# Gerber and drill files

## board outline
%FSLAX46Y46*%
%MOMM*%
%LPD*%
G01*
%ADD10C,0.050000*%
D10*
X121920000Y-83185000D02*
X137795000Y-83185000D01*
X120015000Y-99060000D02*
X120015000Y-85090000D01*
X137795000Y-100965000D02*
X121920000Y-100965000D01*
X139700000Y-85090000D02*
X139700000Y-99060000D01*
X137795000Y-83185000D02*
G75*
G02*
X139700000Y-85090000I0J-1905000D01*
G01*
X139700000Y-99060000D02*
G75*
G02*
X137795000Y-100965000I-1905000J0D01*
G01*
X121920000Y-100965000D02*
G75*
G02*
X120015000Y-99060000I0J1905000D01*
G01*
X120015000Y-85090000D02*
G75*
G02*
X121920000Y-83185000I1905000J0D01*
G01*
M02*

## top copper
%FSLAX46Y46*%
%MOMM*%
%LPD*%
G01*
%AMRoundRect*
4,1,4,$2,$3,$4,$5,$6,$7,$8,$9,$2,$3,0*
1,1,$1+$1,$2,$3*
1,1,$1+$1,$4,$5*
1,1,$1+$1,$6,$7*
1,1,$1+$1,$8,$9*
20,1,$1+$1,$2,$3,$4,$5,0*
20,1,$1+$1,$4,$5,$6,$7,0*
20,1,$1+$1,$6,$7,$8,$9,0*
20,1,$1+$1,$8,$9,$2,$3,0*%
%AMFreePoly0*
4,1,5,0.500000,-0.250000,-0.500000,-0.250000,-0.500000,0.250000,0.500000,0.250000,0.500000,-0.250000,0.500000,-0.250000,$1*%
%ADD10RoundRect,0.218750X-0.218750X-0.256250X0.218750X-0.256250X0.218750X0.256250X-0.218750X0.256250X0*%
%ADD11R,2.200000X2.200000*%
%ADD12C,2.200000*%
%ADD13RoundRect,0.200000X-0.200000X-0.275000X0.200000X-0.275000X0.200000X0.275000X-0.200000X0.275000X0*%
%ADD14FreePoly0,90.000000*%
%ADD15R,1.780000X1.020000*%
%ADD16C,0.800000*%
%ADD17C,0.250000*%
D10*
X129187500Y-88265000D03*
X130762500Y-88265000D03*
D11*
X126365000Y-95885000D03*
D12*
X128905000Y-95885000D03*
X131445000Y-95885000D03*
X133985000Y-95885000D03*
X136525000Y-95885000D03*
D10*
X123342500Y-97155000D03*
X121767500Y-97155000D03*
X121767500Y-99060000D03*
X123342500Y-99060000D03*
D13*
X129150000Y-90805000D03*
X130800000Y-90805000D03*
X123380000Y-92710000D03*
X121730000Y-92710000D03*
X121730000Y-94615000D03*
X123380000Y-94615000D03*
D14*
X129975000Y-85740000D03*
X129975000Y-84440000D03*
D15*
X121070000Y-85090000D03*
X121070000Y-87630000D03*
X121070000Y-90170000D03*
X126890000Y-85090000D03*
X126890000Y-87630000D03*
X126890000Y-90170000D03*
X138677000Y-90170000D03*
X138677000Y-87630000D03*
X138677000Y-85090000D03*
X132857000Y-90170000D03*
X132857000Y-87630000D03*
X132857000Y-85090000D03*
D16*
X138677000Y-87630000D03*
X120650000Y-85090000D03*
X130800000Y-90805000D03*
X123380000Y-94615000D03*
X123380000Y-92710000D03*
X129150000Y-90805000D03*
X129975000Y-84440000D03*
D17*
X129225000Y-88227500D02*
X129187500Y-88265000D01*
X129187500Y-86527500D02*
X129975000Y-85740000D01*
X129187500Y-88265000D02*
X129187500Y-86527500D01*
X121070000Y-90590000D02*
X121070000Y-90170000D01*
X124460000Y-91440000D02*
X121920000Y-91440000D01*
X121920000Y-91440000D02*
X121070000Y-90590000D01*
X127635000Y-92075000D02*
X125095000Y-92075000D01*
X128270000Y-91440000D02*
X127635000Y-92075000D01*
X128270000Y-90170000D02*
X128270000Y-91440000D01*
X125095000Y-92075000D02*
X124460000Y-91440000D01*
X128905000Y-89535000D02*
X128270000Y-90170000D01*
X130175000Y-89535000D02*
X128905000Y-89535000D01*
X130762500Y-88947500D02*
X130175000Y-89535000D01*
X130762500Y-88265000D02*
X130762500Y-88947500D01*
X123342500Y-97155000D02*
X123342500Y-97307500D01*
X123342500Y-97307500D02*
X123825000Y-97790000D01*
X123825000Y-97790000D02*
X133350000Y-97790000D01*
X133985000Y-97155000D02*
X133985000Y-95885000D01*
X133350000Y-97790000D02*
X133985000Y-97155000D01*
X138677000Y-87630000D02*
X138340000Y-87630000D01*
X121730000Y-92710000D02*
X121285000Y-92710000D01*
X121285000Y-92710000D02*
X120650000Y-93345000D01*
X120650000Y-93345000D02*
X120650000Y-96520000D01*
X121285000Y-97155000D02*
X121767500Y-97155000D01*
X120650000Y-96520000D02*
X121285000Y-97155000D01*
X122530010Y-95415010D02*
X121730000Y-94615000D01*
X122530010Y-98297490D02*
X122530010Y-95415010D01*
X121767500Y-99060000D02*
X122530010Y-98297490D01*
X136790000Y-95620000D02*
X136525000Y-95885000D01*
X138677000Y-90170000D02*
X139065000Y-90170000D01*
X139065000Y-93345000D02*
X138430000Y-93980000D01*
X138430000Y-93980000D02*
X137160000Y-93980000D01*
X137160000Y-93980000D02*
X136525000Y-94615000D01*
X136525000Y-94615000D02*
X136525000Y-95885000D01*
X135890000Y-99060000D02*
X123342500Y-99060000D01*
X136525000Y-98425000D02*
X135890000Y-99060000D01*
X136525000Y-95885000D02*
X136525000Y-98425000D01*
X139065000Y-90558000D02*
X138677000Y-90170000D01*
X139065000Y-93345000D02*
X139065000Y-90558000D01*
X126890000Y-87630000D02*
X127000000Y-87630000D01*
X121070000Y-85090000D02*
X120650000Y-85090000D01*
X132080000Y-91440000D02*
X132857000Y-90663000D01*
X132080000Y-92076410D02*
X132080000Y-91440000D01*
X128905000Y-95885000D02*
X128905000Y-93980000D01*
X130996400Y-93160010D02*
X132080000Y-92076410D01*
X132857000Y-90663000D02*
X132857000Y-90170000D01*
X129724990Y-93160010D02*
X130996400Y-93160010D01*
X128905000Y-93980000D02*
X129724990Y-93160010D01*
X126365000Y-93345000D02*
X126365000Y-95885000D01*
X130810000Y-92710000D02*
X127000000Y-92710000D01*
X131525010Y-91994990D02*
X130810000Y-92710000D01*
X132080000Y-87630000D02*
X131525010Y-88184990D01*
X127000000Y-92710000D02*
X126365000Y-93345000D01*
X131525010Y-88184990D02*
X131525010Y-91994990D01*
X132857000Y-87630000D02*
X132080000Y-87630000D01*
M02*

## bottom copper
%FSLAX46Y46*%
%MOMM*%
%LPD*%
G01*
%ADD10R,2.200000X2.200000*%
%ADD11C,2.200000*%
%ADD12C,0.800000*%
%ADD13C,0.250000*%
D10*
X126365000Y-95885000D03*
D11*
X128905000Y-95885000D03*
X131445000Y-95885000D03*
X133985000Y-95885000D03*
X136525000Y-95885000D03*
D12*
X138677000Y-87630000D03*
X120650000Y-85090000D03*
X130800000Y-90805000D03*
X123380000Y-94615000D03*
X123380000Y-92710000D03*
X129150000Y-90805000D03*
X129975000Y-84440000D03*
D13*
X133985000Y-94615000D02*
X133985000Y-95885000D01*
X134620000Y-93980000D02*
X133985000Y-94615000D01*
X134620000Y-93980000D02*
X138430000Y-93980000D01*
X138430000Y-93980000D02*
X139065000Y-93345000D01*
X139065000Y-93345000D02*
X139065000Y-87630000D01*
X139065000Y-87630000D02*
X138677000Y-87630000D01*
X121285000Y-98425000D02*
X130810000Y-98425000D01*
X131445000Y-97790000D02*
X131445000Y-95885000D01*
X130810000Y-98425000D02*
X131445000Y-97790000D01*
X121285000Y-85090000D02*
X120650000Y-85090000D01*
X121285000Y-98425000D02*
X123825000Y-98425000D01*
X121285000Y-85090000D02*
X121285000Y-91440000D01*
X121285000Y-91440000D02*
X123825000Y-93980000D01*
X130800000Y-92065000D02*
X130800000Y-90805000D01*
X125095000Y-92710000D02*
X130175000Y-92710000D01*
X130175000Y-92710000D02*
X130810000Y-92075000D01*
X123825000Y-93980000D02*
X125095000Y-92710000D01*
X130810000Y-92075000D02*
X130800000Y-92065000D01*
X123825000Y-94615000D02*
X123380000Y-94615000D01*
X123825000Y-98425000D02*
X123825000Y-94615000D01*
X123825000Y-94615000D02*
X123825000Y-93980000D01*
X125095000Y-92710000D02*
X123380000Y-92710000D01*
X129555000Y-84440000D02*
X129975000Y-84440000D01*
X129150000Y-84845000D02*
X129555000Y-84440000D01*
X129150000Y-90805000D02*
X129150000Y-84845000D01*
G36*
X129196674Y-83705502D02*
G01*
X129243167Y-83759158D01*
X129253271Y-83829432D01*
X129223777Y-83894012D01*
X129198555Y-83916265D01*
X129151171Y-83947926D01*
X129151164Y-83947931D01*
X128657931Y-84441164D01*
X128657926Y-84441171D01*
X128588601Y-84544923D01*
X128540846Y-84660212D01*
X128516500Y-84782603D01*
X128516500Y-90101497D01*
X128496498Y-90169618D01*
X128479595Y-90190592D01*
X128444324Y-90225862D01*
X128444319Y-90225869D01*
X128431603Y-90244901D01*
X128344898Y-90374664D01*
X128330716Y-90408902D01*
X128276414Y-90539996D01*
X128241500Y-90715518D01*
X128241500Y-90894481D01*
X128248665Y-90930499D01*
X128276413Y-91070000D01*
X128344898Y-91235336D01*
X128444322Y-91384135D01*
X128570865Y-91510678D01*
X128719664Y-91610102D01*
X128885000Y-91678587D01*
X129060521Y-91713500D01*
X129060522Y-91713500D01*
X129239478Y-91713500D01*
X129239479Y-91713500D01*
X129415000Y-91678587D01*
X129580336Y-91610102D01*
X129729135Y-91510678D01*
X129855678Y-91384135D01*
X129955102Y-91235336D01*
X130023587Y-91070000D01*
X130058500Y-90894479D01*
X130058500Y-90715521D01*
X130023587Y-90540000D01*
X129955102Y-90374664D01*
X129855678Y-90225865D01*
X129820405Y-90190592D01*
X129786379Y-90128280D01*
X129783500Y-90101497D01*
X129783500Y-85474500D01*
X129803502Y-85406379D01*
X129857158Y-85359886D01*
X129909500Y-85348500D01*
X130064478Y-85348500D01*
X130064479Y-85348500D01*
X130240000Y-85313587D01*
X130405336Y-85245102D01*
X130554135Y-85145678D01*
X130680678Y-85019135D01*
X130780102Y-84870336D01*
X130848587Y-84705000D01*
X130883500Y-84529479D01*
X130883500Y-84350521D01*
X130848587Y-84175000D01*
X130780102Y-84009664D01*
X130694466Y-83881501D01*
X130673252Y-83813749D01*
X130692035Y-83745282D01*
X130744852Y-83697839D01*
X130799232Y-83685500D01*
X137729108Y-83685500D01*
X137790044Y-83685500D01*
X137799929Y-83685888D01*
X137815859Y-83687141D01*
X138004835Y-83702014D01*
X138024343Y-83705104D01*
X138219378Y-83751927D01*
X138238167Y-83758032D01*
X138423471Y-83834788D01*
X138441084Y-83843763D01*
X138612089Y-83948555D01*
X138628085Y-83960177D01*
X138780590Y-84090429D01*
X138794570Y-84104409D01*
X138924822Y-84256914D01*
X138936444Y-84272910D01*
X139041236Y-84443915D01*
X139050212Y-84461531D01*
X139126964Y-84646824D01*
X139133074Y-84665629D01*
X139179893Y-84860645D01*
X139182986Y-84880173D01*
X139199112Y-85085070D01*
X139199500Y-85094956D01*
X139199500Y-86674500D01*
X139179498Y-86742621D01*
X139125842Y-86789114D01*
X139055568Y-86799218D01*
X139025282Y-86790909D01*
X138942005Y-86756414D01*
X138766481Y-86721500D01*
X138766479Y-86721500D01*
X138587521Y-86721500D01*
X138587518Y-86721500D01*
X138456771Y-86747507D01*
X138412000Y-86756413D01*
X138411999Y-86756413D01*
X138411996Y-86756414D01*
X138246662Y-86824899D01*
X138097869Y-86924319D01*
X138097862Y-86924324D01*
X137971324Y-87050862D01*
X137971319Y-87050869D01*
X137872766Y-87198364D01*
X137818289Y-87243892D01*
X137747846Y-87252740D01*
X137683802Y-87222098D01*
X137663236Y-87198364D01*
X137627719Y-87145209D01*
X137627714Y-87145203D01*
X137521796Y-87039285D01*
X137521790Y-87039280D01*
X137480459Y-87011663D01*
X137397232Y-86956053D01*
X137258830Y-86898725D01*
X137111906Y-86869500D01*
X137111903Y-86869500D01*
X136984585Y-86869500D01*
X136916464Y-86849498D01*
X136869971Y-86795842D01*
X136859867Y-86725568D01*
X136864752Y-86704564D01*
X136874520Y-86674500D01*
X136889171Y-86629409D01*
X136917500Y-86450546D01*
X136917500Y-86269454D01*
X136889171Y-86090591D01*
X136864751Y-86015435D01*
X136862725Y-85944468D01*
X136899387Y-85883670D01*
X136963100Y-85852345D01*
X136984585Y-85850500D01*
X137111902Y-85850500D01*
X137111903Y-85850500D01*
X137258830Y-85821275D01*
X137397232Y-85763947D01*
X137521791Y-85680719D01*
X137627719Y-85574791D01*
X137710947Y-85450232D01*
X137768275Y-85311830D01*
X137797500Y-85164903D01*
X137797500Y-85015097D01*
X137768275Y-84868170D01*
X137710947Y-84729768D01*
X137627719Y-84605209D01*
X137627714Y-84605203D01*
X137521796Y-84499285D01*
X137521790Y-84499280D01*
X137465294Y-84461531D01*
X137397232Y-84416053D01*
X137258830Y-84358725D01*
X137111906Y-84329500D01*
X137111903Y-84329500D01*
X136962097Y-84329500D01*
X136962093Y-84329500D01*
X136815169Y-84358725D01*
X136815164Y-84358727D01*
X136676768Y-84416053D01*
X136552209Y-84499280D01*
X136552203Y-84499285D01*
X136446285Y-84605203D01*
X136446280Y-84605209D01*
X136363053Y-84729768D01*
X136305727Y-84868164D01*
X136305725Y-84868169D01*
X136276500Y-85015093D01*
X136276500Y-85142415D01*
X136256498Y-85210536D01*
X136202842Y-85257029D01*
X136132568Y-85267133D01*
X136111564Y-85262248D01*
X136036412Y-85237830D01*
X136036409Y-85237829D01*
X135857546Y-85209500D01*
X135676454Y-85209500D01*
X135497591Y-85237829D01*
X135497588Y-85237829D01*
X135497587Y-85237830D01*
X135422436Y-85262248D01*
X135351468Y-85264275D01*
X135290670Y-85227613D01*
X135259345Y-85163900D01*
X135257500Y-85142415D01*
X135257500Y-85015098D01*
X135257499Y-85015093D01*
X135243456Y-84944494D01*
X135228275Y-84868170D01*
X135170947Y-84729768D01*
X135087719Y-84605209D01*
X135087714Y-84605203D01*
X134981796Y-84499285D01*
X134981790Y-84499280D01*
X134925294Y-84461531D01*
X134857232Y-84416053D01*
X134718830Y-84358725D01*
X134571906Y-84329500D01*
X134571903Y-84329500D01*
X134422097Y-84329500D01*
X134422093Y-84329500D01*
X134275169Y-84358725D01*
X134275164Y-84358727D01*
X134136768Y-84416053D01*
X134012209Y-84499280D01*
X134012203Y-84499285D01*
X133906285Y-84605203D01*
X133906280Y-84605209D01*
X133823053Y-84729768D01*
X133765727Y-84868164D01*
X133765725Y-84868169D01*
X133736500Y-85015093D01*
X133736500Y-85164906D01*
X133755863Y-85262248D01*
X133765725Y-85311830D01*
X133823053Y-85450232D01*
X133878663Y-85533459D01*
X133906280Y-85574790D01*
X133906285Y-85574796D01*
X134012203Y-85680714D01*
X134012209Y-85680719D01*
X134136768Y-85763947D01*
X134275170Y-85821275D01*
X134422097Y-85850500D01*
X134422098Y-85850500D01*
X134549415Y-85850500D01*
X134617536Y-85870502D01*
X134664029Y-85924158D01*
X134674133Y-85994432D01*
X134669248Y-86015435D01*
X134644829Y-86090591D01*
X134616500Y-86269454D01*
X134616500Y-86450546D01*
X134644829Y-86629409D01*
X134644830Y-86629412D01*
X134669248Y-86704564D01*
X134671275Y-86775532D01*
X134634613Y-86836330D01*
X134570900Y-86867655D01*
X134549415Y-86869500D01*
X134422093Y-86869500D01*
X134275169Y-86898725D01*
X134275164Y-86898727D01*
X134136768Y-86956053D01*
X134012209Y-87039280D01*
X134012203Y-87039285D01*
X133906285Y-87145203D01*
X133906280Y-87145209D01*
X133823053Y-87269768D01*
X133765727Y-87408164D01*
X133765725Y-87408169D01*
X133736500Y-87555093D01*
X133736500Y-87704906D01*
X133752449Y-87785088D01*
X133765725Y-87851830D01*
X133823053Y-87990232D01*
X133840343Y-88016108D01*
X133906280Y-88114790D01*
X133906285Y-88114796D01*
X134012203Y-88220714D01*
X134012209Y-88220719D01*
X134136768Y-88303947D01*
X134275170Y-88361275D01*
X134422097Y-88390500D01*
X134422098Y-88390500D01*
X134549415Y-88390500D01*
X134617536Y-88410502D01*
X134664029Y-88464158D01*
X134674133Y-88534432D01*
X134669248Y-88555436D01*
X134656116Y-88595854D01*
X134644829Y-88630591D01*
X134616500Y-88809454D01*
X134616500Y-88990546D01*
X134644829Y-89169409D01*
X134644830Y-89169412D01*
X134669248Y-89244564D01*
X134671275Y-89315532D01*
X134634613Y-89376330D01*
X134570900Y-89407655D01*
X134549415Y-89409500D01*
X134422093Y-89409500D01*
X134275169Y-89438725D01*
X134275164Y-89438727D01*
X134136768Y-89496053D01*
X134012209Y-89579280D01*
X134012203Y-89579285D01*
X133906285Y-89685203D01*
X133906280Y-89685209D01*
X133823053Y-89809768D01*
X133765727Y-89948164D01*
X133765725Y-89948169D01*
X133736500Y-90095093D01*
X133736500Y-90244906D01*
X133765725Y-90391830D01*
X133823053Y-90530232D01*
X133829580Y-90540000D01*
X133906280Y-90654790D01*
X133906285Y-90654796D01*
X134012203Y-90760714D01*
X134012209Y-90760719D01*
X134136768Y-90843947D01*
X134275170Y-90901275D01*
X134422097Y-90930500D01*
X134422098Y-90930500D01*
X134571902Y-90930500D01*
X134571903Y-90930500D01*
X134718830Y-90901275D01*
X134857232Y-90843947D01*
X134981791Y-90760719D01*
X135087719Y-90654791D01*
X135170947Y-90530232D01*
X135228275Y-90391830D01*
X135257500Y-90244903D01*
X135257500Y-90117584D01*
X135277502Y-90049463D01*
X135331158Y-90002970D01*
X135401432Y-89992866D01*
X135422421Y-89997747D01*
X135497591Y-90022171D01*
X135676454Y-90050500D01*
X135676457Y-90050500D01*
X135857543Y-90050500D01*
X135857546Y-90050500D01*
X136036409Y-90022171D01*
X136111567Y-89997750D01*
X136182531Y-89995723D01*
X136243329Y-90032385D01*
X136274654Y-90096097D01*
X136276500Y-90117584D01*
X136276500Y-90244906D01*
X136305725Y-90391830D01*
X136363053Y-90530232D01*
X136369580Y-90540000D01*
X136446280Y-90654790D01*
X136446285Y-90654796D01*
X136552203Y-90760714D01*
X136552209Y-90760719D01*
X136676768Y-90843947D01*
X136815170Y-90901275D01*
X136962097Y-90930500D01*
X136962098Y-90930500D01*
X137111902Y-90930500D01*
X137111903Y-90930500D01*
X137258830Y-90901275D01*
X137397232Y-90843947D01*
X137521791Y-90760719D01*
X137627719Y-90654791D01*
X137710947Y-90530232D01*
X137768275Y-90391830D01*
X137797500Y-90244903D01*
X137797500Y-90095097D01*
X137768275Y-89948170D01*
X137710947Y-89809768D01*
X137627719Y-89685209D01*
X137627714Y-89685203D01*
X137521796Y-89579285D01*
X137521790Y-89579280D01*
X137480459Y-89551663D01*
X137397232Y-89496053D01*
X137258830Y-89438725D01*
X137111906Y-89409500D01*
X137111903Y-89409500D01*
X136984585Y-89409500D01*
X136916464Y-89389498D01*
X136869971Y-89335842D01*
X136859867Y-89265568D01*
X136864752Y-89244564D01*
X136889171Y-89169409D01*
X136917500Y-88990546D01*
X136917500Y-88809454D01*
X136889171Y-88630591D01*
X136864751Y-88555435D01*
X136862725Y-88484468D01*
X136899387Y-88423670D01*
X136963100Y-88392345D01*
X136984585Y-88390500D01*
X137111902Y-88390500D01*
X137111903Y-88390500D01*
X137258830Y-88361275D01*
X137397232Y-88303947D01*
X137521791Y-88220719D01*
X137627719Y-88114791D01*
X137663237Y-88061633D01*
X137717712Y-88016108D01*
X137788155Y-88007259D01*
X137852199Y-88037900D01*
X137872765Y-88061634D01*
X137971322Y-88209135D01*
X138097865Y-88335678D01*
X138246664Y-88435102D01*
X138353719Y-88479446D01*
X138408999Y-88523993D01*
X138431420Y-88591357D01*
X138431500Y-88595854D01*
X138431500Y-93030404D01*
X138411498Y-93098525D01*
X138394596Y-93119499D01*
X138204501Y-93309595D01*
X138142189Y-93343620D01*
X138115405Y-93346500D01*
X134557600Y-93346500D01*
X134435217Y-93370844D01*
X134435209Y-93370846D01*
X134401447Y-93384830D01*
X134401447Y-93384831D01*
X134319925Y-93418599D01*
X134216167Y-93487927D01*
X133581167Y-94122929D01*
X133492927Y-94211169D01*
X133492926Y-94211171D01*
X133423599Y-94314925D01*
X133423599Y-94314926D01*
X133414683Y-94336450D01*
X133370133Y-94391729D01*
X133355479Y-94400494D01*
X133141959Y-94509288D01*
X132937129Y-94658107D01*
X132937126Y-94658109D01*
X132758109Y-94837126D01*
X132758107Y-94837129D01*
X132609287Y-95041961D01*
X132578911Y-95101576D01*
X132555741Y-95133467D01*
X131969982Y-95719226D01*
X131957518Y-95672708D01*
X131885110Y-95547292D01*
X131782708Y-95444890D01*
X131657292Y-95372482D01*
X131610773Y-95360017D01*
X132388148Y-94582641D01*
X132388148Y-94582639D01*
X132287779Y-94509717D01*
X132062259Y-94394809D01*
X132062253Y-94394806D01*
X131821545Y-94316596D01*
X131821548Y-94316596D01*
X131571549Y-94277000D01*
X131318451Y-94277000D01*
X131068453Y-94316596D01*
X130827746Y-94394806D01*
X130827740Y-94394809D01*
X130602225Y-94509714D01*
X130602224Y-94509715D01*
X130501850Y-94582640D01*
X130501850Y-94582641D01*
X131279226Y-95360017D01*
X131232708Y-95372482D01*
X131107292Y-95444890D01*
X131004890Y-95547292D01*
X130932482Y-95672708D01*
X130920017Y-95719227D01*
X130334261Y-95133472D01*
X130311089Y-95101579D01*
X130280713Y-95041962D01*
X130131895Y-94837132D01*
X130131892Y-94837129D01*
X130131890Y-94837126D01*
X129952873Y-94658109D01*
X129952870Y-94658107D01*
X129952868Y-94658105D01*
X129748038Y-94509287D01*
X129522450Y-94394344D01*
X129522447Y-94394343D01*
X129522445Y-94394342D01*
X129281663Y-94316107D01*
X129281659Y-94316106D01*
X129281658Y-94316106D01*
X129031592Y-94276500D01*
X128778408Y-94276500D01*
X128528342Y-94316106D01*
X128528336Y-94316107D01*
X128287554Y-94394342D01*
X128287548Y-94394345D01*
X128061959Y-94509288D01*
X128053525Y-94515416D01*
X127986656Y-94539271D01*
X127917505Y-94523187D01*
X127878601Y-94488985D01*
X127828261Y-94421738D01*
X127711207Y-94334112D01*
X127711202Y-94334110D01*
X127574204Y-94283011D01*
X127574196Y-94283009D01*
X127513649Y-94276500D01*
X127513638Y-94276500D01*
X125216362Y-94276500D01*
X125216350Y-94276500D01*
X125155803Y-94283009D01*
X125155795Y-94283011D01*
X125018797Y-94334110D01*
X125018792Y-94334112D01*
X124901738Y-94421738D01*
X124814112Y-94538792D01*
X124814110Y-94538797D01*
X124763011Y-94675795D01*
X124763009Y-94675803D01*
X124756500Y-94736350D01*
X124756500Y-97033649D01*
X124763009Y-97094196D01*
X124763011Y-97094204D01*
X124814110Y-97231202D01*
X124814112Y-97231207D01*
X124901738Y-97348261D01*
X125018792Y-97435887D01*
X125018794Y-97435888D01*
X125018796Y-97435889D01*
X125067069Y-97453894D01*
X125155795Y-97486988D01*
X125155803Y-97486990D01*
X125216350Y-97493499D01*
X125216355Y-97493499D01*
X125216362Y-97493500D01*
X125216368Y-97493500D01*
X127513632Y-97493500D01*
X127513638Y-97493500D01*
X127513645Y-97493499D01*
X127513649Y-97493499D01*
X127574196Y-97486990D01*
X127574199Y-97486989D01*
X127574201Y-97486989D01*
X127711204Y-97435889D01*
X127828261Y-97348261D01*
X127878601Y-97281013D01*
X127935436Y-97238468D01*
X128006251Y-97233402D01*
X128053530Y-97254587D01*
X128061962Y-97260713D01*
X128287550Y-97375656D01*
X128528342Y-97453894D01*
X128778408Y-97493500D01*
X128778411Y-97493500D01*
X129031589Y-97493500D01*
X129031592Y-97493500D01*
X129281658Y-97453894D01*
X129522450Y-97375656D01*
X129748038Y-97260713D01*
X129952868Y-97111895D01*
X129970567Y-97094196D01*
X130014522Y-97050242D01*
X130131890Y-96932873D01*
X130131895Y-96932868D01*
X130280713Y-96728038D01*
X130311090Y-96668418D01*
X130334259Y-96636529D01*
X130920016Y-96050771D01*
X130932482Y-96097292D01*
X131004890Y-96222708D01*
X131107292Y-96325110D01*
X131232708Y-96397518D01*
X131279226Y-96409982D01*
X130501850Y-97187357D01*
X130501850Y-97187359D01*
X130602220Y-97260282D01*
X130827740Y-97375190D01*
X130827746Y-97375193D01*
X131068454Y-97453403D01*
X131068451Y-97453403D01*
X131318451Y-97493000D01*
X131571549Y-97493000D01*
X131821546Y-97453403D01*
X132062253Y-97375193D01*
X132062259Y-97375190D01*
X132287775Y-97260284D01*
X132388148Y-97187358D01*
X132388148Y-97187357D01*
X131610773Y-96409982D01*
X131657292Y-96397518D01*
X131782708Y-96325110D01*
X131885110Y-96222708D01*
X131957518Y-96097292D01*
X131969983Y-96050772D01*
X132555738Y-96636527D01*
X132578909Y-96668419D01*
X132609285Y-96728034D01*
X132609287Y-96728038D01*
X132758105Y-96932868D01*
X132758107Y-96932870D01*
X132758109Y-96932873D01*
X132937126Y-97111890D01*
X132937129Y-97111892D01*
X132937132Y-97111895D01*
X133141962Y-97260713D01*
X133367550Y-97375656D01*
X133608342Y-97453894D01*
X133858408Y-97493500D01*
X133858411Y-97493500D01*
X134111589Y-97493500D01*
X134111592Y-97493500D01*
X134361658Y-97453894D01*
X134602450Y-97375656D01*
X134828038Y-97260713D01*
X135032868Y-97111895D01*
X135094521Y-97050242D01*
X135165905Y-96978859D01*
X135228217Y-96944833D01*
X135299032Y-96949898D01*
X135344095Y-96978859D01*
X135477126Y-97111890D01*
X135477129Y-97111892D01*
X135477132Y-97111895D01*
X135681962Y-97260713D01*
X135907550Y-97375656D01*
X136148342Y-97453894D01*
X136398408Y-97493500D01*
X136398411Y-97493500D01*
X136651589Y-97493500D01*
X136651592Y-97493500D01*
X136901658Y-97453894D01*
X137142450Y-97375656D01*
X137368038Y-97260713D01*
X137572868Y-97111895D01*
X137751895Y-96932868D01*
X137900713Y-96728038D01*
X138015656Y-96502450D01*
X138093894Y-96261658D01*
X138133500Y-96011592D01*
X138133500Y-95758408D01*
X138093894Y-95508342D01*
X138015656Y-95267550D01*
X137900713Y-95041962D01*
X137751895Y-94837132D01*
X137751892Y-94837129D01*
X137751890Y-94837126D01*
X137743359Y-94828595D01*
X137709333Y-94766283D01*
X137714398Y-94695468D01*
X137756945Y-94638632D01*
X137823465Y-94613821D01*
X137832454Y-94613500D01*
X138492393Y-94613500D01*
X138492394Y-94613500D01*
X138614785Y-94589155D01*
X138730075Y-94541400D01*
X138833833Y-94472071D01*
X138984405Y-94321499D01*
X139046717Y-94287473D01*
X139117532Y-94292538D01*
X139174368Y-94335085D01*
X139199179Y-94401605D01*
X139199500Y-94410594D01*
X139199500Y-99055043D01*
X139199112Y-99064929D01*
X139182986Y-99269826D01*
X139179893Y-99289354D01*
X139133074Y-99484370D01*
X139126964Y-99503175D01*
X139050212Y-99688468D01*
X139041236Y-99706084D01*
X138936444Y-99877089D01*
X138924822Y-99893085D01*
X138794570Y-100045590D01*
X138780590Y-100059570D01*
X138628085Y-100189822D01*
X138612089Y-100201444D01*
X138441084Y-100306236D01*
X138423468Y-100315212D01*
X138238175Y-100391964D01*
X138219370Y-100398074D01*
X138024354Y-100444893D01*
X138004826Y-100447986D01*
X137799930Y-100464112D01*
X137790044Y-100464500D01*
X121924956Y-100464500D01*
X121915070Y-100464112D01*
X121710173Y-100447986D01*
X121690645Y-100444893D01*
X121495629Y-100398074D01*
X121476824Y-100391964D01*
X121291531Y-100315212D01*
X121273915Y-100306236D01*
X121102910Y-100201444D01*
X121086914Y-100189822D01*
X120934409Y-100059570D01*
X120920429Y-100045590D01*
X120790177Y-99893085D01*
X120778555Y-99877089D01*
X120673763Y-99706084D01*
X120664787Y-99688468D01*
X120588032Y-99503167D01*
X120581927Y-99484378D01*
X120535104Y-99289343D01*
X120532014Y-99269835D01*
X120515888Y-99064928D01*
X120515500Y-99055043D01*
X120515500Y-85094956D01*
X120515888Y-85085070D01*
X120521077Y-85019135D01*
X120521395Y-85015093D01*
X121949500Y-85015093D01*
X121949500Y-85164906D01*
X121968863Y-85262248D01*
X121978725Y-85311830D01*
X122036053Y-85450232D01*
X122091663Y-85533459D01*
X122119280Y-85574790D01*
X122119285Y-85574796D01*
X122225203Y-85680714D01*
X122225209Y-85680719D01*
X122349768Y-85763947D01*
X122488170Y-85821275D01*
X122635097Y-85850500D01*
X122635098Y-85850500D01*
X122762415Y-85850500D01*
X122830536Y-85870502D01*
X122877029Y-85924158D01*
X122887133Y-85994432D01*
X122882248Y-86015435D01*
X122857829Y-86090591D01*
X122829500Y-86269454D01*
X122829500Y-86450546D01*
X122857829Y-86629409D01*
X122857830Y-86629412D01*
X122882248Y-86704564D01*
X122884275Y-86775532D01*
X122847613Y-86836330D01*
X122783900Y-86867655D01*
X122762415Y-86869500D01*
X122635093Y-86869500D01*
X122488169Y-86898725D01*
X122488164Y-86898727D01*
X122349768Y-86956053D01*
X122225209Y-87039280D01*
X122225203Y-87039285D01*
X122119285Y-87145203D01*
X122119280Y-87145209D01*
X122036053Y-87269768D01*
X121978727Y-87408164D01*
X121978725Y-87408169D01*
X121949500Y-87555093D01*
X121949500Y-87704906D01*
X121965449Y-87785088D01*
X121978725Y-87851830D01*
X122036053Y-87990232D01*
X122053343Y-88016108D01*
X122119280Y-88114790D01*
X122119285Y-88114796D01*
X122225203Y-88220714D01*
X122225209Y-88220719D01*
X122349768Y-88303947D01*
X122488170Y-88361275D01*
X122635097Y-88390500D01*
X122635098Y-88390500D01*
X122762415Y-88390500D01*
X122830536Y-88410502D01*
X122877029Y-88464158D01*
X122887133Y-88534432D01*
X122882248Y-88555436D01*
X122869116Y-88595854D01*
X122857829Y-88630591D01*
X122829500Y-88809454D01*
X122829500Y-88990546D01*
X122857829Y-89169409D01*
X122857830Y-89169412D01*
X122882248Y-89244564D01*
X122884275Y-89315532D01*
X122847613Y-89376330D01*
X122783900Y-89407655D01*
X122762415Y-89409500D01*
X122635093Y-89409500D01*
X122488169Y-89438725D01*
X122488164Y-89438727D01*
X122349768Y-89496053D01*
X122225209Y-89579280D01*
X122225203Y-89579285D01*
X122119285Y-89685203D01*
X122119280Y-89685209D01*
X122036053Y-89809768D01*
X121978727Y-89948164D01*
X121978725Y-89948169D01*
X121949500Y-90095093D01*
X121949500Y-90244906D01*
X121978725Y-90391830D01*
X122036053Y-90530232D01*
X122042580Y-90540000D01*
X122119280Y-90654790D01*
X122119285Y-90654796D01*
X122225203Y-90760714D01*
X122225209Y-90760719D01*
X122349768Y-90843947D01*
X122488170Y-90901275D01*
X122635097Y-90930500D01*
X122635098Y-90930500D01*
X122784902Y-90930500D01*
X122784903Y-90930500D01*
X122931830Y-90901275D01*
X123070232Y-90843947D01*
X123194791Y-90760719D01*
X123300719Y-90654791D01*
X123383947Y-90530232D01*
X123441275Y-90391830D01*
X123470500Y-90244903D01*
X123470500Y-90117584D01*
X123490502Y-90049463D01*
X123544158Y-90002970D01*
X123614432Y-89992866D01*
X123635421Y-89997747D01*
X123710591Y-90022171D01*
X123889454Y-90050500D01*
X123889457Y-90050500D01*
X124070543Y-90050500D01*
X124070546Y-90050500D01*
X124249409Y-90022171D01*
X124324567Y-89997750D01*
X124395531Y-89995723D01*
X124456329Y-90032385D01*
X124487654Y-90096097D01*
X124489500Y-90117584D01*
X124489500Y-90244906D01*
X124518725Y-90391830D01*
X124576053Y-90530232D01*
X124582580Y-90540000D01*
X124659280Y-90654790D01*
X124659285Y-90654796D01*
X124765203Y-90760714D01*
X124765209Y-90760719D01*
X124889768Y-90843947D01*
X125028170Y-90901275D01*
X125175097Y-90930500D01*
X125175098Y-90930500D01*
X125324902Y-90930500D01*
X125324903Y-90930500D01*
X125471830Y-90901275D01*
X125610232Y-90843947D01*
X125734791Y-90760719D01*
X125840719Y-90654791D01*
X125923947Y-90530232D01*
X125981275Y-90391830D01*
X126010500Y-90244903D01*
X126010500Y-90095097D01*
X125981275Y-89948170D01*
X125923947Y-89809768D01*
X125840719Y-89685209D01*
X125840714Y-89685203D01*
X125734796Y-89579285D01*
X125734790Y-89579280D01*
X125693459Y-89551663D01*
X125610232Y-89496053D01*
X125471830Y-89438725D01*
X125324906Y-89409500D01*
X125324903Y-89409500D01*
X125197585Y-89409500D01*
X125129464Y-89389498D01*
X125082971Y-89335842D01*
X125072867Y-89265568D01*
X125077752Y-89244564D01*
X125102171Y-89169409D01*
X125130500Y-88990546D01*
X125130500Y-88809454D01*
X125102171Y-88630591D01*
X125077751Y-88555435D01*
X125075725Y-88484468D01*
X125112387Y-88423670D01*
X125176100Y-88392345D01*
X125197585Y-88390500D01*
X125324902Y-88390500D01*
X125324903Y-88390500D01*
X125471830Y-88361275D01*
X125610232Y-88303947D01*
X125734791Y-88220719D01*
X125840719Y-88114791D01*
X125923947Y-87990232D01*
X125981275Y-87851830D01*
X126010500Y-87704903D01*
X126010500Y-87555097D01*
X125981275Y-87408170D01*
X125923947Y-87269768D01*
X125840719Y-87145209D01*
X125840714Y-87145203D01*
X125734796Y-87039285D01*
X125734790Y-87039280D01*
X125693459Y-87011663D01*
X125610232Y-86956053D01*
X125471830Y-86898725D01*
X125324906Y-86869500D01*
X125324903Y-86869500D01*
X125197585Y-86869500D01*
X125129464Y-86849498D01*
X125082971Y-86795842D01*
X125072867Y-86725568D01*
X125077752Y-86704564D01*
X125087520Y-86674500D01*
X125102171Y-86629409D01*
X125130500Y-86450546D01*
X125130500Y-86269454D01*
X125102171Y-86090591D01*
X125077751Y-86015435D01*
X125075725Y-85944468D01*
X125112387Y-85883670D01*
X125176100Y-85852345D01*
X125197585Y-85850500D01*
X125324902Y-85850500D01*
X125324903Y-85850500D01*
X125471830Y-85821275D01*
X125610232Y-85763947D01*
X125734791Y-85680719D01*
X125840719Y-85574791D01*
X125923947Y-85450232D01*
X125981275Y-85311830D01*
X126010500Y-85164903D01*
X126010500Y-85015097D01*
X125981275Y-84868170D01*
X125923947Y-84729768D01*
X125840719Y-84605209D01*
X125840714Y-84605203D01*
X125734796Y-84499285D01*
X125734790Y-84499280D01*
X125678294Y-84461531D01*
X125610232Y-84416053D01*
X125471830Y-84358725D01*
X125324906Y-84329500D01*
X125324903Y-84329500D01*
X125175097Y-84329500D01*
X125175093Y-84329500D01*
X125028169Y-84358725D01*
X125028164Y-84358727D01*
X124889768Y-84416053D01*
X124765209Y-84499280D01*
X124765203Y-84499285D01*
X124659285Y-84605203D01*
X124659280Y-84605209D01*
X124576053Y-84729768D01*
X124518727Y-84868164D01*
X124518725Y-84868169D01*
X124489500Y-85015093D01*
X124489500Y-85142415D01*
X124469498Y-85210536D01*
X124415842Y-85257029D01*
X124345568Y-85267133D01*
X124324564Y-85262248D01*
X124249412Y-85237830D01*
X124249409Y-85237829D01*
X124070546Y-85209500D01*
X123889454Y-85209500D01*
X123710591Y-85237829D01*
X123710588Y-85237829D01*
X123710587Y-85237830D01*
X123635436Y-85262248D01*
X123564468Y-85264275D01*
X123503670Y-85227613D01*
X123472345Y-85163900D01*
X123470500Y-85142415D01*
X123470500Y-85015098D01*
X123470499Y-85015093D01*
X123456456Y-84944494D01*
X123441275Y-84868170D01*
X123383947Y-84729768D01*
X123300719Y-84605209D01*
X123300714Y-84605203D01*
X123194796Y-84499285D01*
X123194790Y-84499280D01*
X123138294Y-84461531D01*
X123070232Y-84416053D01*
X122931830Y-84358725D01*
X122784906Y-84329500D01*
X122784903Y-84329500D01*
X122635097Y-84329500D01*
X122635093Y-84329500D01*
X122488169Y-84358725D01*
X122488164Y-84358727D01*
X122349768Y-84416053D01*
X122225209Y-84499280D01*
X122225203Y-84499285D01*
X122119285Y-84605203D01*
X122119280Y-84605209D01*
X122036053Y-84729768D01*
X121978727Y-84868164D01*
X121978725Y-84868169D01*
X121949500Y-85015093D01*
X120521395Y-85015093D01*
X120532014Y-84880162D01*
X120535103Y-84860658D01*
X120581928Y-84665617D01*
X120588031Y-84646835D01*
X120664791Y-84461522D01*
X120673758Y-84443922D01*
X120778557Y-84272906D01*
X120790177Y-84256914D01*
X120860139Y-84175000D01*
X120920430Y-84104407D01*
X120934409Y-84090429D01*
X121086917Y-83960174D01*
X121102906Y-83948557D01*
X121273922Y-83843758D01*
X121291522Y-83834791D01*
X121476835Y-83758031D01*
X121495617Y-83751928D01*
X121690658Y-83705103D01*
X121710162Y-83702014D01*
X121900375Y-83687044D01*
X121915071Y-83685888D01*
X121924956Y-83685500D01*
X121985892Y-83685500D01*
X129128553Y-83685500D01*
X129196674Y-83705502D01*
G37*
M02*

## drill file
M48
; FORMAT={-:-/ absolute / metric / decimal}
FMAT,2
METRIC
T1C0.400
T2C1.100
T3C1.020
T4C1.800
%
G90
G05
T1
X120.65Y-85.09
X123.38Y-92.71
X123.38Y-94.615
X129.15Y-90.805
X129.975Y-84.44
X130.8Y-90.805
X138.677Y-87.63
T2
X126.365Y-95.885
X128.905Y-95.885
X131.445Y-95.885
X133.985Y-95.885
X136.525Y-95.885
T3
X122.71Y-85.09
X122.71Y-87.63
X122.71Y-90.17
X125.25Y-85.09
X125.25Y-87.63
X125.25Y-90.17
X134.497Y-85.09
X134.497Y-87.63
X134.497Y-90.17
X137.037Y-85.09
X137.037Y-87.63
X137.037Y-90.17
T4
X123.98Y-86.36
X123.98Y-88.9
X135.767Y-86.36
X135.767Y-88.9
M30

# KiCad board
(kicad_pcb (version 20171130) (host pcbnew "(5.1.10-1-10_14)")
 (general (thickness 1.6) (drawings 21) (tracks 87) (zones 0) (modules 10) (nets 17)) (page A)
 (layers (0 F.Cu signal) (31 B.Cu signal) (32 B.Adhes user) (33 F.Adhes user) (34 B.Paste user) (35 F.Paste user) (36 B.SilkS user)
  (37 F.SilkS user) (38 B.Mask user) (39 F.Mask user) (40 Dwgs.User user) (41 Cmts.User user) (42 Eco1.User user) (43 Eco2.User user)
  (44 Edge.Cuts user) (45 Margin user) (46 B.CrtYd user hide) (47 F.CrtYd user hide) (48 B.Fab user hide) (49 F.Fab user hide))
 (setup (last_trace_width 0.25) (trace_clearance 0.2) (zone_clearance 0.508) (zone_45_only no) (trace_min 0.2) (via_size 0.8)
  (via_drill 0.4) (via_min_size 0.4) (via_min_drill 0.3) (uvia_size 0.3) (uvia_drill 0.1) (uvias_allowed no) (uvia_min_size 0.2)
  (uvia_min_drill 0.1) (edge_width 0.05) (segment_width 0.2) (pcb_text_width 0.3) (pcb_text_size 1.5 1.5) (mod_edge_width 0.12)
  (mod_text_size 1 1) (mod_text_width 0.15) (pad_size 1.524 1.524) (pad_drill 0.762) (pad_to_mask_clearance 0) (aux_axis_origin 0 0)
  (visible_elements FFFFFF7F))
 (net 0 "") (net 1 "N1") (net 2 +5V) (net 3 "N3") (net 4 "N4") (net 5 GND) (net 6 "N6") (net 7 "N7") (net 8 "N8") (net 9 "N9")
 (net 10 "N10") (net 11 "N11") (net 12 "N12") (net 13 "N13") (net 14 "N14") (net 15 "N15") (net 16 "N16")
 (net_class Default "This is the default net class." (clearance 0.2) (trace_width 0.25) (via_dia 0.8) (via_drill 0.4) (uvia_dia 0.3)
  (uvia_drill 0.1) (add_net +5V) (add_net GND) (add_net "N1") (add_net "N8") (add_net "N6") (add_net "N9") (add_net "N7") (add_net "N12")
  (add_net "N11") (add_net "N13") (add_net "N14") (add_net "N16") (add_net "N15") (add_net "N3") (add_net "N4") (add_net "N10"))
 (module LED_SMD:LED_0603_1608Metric (layer F.Cu) (at 129.975 88.265)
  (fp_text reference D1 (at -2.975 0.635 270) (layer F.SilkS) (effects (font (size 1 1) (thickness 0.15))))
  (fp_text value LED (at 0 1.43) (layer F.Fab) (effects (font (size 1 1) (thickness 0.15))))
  (pad 1 smd roundrect (at -0.7875 0) (size 0.875 0.95) (layers F.Cu F.Paste F.Mask) (roundrect_rratio 0.25) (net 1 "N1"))
  (pad 2 smd roundrect (at 0.7875 0) (size 0.875 0.95) (layers F.Cu F.Paste F.Mask) (roundrect_rratio 0.25) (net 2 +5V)))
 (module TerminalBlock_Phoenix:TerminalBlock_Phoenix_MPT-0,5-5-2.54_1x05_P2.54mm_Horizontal (layer F.Cu) (at 126.365 95.885)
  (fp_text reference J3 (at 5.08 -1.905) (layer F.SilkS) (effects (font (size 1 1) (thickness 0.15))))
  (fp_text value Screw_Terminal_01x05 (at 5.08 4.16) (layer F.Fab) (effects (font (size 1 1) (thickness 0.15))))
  (pad 1 thru_hole rect (at 0 0) (size 2.2 2.2) (drill 1.1) (layers *.Cu *.Mask) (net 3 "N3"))
  (pad 2 thru_hole circle (at 2.54 0) (size 2.2 2.2) (drill 1.1) (layers *.Cu *.Mask) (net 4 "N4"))
  (pad 3 thru_hole circle (at 5.08 0) (size 2.2 2.2) (drill 1.1) (layers *.Cu *.Mask) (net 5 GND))
  (pad 4 thru_hole circle (at 7.62 0) (size 2.2 2.2) (drill 1.1) (layers *.Cu *.Mask) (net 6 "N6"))
  (pad 5 thru_hole circle (at 10.16 0) (size 2.2 2.2) (drill 1.1) (layers *.Cu *.Mask) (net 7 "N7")))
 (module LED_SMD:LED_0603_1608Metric (layer F.Cu) (at 122.555 97.155)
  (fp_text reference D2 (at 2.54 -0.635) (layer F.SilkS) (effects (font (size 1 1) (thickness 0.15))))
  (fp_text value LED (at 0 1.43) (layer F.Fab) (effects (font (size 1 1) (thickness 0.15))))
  (pad 2 smd roundrect (at 0.7875 0) (size 0.875 0.95) (layers F.Cu F.Paste F.Mask) (roundrect_rratio 0.25) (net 6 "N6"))
  (pad 1 smd roundrect (at -0.7875 0) (size 0.875 0.95) (layers F.Cu F.Paste F.Mask) (roundrect_rratio 0.25) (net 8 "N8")))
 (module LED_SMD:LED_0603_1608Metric (layer F.Cu) (at 122.555 99.06)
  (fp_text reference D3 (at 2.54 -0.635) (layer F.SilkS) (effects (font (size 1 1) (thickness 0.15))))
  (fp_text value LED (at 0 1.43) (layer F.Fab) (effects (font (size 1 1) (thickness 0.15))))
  (pad 1 smd roundrect (at -0.7875 0) (size 0.875 0.95) (layers F.Cu F.Paste F.Mask) (roundrect_rratio 0.25) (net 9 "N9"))
  (pad 2 smd roundrect (at 0.7875 0) (size 0.875 0.95) (layers F.Cu F.Paste F.Mask) (roundrect_rratio 0.25) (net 7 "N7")))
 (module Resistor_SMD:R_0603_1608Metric (layer F.Cu) (at 129.975 90.805)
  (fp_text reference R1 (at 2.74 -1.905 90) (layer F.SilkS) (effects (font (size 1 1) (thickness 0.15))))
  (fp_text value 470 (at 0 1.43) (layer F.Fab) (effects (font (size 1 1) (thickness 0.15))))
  (pad 1 smd roundrect (at -0.825 0) (size 0.8 0.95) (layers F.Cu F.Paste F.Mask) (roundrect_rratio 0.25) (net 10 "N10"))
  (pad 2 smd roundrect (at 0.825 0) (size 0.8 0.95) (layers F.Cu F.Paste F.Mask) (roundrect_rratio 0.25) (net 5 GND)))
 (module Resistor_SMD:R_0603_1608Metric (layer F.Cu) (at 122.555 92.71)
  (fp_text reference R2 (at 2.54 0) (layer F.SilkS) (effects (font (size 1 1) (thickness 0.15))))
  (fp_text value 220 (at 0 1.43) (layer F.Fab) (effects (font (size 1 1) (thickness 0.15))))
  (pad 2 smd roundrect (at 0.825 0) (size 0.8 0.95) (layers F.Cu F.Paste F.Mask) (roundrect_rratio 0.25) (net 5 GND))
  (pad 1 smd roundrect (at -0.825 0) (size 0.8 0.95) (layers F.Cu F.Paste F.Mask) (roundrect_rratio 0.25) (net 8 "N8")))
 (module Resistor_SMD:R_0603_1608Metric (layer F.Cu) (at 122.555 94.615)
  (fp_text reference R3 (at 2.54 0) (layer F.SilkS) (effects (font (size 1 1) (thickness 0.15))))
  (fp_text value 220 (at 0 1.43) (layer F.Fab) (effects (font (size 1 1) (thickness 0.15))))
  (pad 1 smd roundrect (at -0.825 0) (size 0.8 0.95) (layers F.Cu F.Paste F.Mask) (roundrect_rratio 0.25) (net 9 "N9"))
  (pad 2 smd roundrect (at 0.825 0) (size 0.8 0.95) (layers F.Cu F.Paste F.Mask) (roundrect_rratio 0.25) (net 5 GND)))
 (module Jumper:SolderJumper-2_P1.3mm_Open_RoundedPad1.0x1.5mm (layer F.Cu) (at 129.975 85.09 90)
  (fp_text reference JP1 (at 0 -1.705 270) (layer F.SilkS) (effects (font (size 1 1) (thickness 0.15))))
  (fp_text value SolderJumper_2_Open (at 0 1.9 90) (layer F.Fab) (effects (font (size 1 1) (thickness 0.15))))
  (pad 1 smd custom (at -0.65 0 90) (size 1 0.5) (layers F.Cu F.Mask) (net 1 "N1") (zone_connect 2)
   (options (clearance outline) (anchor rect)) (primitives))
  (pad 2 smd custom (at 0.65 0 90) (size 1 0.5) (layers F.Cu F.Mask) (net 10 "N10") (zone_connect 2)
   (options (clearance outline) (anchor rect)) (primitives)))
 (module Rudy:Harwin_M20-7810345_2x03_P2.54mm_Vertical (layer F.Cu) (at 123.98 87.63)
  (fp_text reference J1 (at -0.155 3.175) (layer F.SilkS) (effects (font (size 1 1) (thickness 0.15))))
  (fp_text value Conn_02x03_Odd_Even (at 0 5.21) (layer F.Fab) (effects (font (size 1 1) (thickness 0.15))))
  (pad "" np_thru_hole circle (at 0 -1.27) (size 1.8 1.8) (drill 1.8) (layers *.Cu *.Mask))
  (pad "" np_thru_hole circle (at 0 1.27) (size 1.8 1.8) (drill 1.8) (layers *.Cu *.Mask))
  (pad "" np_thru_hole circle (at -1.27 -2.54) (size 1.02 1.02) (drill 1.02) (layers *.Cu *.Mask))
  (pad "" np_thru_hole circle (at -1.27 0) (size 1.02 1.02) (drill 1.02) (layers *.Cu *.Mask))
  (pad "" np_thru_hole circle (at -1.27 2.54) (size 1.02 1.02) (drill 1.02) (layers *.Cu *.Mask))
  (pad "" np_thru_hole circle (at 1.27 -2.54) (size 1.02 1.02) (drill 1.02) (layers *.Cu *.Mask))
  (pad "" np_thru_hole circle (at 1.27 0) (size 1.02 1.02) (drill 1.02) (layers *.Cu *.Mask))
  (pad "" np_thru_hole circle (at 1.27 2.54) (size 1.02 1.02) (drill 1.02) (layers *.Cu *.Mask))
  (pad 1 smd rect (at -2.91 -2.54) (size 1.78 1.02) (layers F.Cu F.Paste F.Mask) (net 5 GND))
  (pad 3 smd rect (at -2.91 0) (size 1.78 1.02) (layers F.Cu F.Paste F.Mask) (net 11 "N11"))
  (pad 5 smd rect (at -2.91 2.54) (size 1.78 1.02) (layers F.Cu F.Paste F.Mask) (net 2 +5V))
  (pad 2 smd rect (at 2.91 -2.54) (size 1.78 1.02) (layers F.Cu F.Paste F.Mask) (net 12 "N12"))
  (pad 4 smd rect (at 2.91 0) (size 1.78 1.02) (layers F.Cu F.Paste F.Mask) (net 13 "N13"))
  (pad 6 smd rect (at 2.91 2.54) (size 1.78 1.02) (layers F.Cu F.Paste F.Mask) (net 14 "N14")))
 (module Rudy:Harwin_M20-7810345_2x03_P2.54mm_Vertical (layer F.Cu) (at 135.767 87.63)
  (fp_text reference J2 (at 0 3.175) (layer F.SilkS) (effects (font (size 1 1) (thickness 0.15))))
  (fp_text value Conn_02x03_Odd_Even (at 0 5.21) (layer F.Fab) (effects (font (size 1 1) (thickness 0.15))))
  (pad 6 smd rect (at 2.91 2.54) (size 1.78 1.02) (layers F.Cu F.Paste F.Mask) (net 7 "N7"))
  (pad 4 smd rect (at 2.91 0) (size 1.78 1.02) (layers F.Cu F.Paste F.Mask) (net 6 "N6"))
  (pad 2 smd rect (at 2.91 -2.54) (size 1.78 1.02) (layers F.Cu F.Paste F.Mask) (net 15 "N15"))
  (pad 5 smd rect (at -2.91 2.54) (size 1.78 1.02) (layers F.Cu F.Paste F.Mask) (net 4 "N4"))
  (pad 3 smd rect (at -2.91 0) (size 1.78 1.02) (layers F.Cu F.Paste F.Mask) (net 3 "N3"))
  (pad 1 smd rect (at -2.91 -2.54) (size 1.78 1.02) (layers F.Cu F.Paste F.Mask) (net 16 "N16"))
  (pad "" np_thru_hole circle (at 1.27 2.54) (size 1.02 1.02) (drill 1.02) (layers *.Cu *.Mask))
  (pad "" np_thru_hole circle (at 1.27 0) (size 1.02 1.02) (drill 1.02) (layers *.Cu *.Mask))
  (pad "" np_thru_hole circle (at 1.27 -2.54) (size 1.02 1.02) (drill 1.02) (layers *.Cu *.Mask))
  (pad "" np_thru_hole circle (at -1.27 2.54) (size 1.02 1.02) (drill 1.02) (layers *.Cu *.Mask))
  (pad "" np_thru_hole circle (at -1.27 0) (size 1.02 1.02) (drill 1.02) (layers *.Cu *.Mask))
  (pad "" np_thru_hole circle (at -1.27 -2.54) (size 1.02 1.02) (drill 1.02) (layers *.Cu *.Mask))
  (pad "" np_thru_hole circle (at 0 1.27) (size 1.8 1.8) (drill 1.8) (layers *.Cu *.Mask))
  (pad "" np_thru_hole circle (at 0 -1.27) (size 1.8 1.8) (drill 1.8) (layers *.Cu *.Mask)))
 (gr_line (start 121.92 83.185) (end 137.795 83.185) (layer Edge.Cuts) (width 0.05))
 (gr_line (start 120.015 99.06) (end 120.015 85.09) (layer Edge.Cuts) (width 0.05))
 (gr_line (start 137.795 100.965) (end 121.92 100.965) (layer Edge.Cuts) (width 0.05))
 (gr_line (start 139.7 85.09) (end 139.7 99.06) (layer Edge.Cuts) (width 0.05))
 (gr_arc (start 137.795 85.09) (end 139.7 85.09) (angle -90) (layer Edge.Cuts) (width 0.05))
 (gr_arc (start 137.795 99.06) (end 137.795 100.965) (angle -90) (layer Edge.Cuts) (width 0.05))
 (gr_arc (start 121.92 99.06) (end 120.015 99.06) (angle -90) (layer Edge.Cuts) (width 0.05))
 (gr_arc (start 121.92 85.09) (end 121.92 83.185) (angle -90) (layer Edge.Cuts) (width 0.05))
 (segment (start 129.225 88.2275) (end 129.1875 88.265) (width 0.25) (layer F.Cu) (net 1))
 (segment (start 129.1875 86.5275) (end 129.975 85.74) (width 0.25) (layer F.Cu) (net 1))
 (segment (start 129.1875 88.265) (end 129.1875 86.5275) (width 0.25) (layer F.Cu) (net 1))
 (segment (start 121.07 90.59) (end 121.07 90.17) (width 0.25) (layer F.Cu) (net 2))
 (segment (start 124.46 91.44) (end 121.92 91.44) (width 0.25) (layer F.Cu) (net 2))
 (segment (start 121.92 91.44) (end 121.07 90.59) (width 0.25) (layer F.Cu) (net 2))
 (segment (start 127.635 92.075) (end 125.095 92.075) (width 0.25) (layer F.Cu) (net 2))
 (segment (start 128.27 91.44) (end 127.635 92.075) (width 0.25) (layer F.Cu) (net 2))
 (segment (start 128.27 90.17) (end 128.27 91.44) (width 0.25) (layer F.Cu) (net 2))
 (segment (start 125.095 92.075) (end 124.46 91.44) (width 0.25) (layer F.Cu) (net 2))
 (segment (start 128.905 89.535) (end 128.27 90.17) (width 0.25) (layer F.Cu) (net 2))
 (segment (start 130.175 89.535) (end 128.905 89.535) (width 0.25) (layer F.Cu) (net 2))
 (segment (start 130.7625 88.9475) (end 130.175 89.535) (width 0.25) (layer F.Cu) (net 2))
 (segment (start 130.7625 88.265) (end 130.7625 88.9475) (width 0.25) (layer F.Cu) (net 2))
 (segment (start 133.985 94.615) (end 133.985 95.885) (width 0.25) (layer B.Cu) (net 6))
 (segment (start 134.62 93.98) (end 133.985 94.615) (width 0.25) (layer B.Cu) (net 6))
 (segment (start 123.3425 97.155) (end 123.3425 97.3075) (width 0.25) (layer F.Cu) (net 6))
 (segment (start 123.3425 97.3075) (end 123.825 97.79) (width 0.25) (layer F.Cu) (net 6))
 (segment (start 123.825 97.79) (end 133.35 97.79) (width 0.25) (layer F.Cu) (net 6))
 (segment (start 133.985 97.155) (end 133.985 95.885) (width 0.25) (layer F.Cu) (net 6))
 (segment (start 133.35 97.79) (end 133.985 97.155) (width 0.25) (layer F.Cu) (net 6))
 (segment (start 138.677 87.63) (end 138.34 87.63) (width 0.25) (layer F.Cu) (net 6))
 (segment (start 134.62 93.98) (end 138.43 93.98) (width 0.25) (layer B.Cu) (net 6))
 (segment (start 138.43 93.98) (end 139.065 93.345) (width 0.25) (layer B.Cu) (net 6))
 (segment (start 139.065 93.345) (end 139.065 87.63) (width 0.25) (layer B.Cu) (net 6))
 (via (at 138.677 87.63) (size 0.8) (drill 0.4) (layers F.Cu B.Cu) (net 6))
 (segment (start 139.065 87.63) (end 138.677 87.63) (width 0.25) (layer B.Cu) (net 6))
 (segment (start 121.73 92.71) (end 121.285 92.71) (width 0.25) (layer F.Cu) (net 8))
 (segment (start 121.285 92.71) (end 120.65 93.345) (width 0.25) (layer F.Cu) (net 8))
 (segment (start 120.65 93.345) (end 120.65 96.52) (width 0.25) (layer F.Cu) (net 8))
 (segment (start 121.285 97.155) (end 121.7675 97.155) (width 0.25) (layer F.Cu) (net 8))
 (segment (start 120.65 96.52) (end 121.285 97.155) (width 0.25) (layer F.Cu) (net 8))
 (segment (start 122.53001 95.41501) (end 121.73 94.615) (width 0.25) (layer F.Cu) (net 9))
 (segment (start 122.53001 98.29749) (end 122.53001 95.41501) (width 0.25) (layer F.Cu) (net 9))
 (segment (start 121.7675 99.06) (end 122.53001 98.29749) (width 0.25) (layer F.Cu) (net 9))
 (segment (start 136.79 95.62) (end 136.525 95.885) (width 0.25) (layer F.Cu) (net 7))
 (segment (start 138.677 90.17) (end 139.065 90.17) (width 0.25) (layer F.Cu) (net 7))
 (segment (start 139.065 93.345) (end 138.43 93.98) (width 0.25) (layer F.Cu) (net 7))
 (segment (start 138.43 93.98) (end 137.16 93.98) (width 0.25) (layer F.Cu) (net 7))
 (segment (start 137.16 93.98) (end 136.525 94.615) (width 0.25) (layer F.Cu) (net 7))
 (segment (start 136.525 94.615) (end 136.525 95.885) (width 0.25) (layer F.Cu) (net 7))
 (segment (start 135.89 99.06) (end 123.3425 99.06) (width 0.25) (layer F.Cu) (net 7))
 (segment (start 136.525 98.425) (end 135.89 99.06) (width 0.25) (layer F.Cu) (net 7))
 (segment (start 136.525 95.885) (end 136.525 98.425) (width 0.25) (layer F.Cu) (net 7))
 (segment (start 139.065 90.558) (end 138.677 90.17) (width 0.25) (layer F.Cu) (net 7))
 (segment (start 139.065 93.345) (end 139.065 90.558) (width 0.25) (layer F.Cu) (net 7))
 (segment (start 126.89 87.63) (end 127 87.63) (width 0.25) (layer F.Cu) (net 13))
 (via (at 120.65 85.09) (size 0.8) (drill 0.4) (layers F.Cu B.Cu) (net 5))
 (segment (start 121.07 85.09) (end 120.65 85.09) (width 0.25) (layer F.Cu) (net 5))
 (segment (start 121.285 98.425) (end 130.81 98.425) (width 0.25) (layer B.Cu) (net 5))
 (segment (start 131.445 97.79) (end 131.445 95.885) (width 0.25) (layer B.Cu) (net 5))
 (segment (start 130.81 98.425) (end 131.445 97.79) (width 0.25) (layer B.Cu) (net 5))
 (segment (start 121.285 85.09) (end 120.65 85.09) (width 0.25) (layer B.Cu) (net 5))
 (segment (start 121.285 98.425) (end 123.825 98.425) (width 0.25) (layer B.Cu) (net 5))
 (segment (start 121.285 85.09) (end 121.285 91.44) (width 0.25) (layer B.Cu) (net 5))
 (segment (start 121.285 91.44) (end 123.825 93.98) (width 0.25) (layer B.Cu) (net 5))
 (segment (start 130.8 92.065) (end 130.8 90.805) (width 0.25) (layer B.Cu) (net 5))
 (via (at 130.8 90.805) (size 0.8) (drill 0.4) (layers F.Cu B.Cu) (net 5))
 (segment (start 125.095 92.71) (end 130.175 92.71) (width 0.25) (layer B.Cu) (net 5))
 (segment (start 130.175 92.71) (end 130.81 92.075) (width 0.25) (layer B.Cu) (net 5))
 (segment (start 123.825 93.98) (end 125.095 92.71) (width 0.25) (layer B.Cu) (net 5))
 (segment (start 130.81 92.075) (end 130.8 92.065) (width 0.25) (layer B.Cu) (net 5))
 (via (at 123.38 94.615) (size 0.8) (drill 0.4) (layers F.Cu B.Cu) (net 5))
 (segment (start 123.825 94.615) (end 123.38 94.615) (width 0.25) (layer B.Cu) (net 5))
 (segment (start 123.825 98.425) (end 123.825 94.615) (width 0.25) (layer B.Cu) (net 5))
 (segment (start 123.825 94.615) (end 123.825 93.98) (width 0.25) (layer B.Cu) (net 5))
 (via (at 123.38 92.71) (size 0.8) (drill 0.4) (layers F.Cu B.Cu) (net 5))
 (segment (start 125.095 92.71) (end 123.38 92.71) (width 0.25) (layer B.Cu) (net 5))
 (segment (start 132.08 91.44) (end 132.857 90.663) (width 0.25) (layer F.Cu) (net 4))
 (segment (start 132.08 92.07641) (end 132.08 91.44) (width 0.25) (layer F.Cu) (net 4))
 (segment (start 128.905 95.885) (end 128.905 93.98) (width 0.25) (layer F.Cu) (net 4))
 (segment (start 130.9964 93.16001) (end 132.08 92.07641) (width 0.25) (layer F.Cu) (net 4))
 (segment (start 132.857 90.663) (end 132.857 90.17) (width 0.25) (layer F.Cu) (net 4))
 (segment (start 129.72499 93.16001) (end 130.9964 93.16001) (width 0.25) (layer F.Cu) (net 4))
 (segment (start 128.905 93.98) (end 129.72499 93.16001) (width 0.25) (layer F.Cu) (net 4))
 (segment (start 126.365 93.345) (end 126.365 95.885) (width 0.25) (layer F.Cu) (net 3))
 (segment (start 130.81 92.71) (end 127 92.71) (width 0.25) (layer F.Cu) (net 3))
 (segment (start 131.52501 91.99499) (end 130.81 92.71) (width 0.25) (layer F.Cu) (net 3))
 (segment (start 132.08 87.63) (end 131.52501 88.18499) (width 0.25) (layer F.Cu) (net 3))
 (segment (start 127 92.71) (end 126.365 93.345) (width 0.25) (layer F.Cu) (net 3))
 (segment (start 131.52501 88.18499) (end 131.52501 91.99499) (width 0.25) (layer F.Cu) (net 3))
 (segment (start 132.857 87.63) (end 132.08 87.63) (width 0.25) (layer F.Cu) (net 3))
 (via (at 129.15 90.805) (size 0.8) (drill 0.4) (layers F.Cu B.Cu) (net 10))
 (segment (start 129.555 84.44) (end 129.975 84.44) (width 0.25) (layer B.Cu) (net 10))
 (segment (start 129.15 84.845) (end 129.555 84.44) (width 0.25) (layer B.Cu) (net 10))
 (segment (start 129.15 90.805) (end 129.15 84.845) (width 0.25) (layer B.Cu) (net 10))
 (via (at 129.975 84.44) (size 0.8) (drill 0.4) (layers F.Cu B.Cu) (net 10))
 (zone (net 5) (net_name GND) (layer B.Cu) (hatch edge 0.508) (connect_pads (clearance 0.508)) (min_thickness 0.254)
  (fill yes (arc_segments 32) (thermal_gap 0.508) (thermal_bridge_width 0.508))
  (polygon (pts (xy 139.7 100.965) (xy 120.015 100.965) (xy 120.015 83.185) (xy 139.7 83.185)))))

